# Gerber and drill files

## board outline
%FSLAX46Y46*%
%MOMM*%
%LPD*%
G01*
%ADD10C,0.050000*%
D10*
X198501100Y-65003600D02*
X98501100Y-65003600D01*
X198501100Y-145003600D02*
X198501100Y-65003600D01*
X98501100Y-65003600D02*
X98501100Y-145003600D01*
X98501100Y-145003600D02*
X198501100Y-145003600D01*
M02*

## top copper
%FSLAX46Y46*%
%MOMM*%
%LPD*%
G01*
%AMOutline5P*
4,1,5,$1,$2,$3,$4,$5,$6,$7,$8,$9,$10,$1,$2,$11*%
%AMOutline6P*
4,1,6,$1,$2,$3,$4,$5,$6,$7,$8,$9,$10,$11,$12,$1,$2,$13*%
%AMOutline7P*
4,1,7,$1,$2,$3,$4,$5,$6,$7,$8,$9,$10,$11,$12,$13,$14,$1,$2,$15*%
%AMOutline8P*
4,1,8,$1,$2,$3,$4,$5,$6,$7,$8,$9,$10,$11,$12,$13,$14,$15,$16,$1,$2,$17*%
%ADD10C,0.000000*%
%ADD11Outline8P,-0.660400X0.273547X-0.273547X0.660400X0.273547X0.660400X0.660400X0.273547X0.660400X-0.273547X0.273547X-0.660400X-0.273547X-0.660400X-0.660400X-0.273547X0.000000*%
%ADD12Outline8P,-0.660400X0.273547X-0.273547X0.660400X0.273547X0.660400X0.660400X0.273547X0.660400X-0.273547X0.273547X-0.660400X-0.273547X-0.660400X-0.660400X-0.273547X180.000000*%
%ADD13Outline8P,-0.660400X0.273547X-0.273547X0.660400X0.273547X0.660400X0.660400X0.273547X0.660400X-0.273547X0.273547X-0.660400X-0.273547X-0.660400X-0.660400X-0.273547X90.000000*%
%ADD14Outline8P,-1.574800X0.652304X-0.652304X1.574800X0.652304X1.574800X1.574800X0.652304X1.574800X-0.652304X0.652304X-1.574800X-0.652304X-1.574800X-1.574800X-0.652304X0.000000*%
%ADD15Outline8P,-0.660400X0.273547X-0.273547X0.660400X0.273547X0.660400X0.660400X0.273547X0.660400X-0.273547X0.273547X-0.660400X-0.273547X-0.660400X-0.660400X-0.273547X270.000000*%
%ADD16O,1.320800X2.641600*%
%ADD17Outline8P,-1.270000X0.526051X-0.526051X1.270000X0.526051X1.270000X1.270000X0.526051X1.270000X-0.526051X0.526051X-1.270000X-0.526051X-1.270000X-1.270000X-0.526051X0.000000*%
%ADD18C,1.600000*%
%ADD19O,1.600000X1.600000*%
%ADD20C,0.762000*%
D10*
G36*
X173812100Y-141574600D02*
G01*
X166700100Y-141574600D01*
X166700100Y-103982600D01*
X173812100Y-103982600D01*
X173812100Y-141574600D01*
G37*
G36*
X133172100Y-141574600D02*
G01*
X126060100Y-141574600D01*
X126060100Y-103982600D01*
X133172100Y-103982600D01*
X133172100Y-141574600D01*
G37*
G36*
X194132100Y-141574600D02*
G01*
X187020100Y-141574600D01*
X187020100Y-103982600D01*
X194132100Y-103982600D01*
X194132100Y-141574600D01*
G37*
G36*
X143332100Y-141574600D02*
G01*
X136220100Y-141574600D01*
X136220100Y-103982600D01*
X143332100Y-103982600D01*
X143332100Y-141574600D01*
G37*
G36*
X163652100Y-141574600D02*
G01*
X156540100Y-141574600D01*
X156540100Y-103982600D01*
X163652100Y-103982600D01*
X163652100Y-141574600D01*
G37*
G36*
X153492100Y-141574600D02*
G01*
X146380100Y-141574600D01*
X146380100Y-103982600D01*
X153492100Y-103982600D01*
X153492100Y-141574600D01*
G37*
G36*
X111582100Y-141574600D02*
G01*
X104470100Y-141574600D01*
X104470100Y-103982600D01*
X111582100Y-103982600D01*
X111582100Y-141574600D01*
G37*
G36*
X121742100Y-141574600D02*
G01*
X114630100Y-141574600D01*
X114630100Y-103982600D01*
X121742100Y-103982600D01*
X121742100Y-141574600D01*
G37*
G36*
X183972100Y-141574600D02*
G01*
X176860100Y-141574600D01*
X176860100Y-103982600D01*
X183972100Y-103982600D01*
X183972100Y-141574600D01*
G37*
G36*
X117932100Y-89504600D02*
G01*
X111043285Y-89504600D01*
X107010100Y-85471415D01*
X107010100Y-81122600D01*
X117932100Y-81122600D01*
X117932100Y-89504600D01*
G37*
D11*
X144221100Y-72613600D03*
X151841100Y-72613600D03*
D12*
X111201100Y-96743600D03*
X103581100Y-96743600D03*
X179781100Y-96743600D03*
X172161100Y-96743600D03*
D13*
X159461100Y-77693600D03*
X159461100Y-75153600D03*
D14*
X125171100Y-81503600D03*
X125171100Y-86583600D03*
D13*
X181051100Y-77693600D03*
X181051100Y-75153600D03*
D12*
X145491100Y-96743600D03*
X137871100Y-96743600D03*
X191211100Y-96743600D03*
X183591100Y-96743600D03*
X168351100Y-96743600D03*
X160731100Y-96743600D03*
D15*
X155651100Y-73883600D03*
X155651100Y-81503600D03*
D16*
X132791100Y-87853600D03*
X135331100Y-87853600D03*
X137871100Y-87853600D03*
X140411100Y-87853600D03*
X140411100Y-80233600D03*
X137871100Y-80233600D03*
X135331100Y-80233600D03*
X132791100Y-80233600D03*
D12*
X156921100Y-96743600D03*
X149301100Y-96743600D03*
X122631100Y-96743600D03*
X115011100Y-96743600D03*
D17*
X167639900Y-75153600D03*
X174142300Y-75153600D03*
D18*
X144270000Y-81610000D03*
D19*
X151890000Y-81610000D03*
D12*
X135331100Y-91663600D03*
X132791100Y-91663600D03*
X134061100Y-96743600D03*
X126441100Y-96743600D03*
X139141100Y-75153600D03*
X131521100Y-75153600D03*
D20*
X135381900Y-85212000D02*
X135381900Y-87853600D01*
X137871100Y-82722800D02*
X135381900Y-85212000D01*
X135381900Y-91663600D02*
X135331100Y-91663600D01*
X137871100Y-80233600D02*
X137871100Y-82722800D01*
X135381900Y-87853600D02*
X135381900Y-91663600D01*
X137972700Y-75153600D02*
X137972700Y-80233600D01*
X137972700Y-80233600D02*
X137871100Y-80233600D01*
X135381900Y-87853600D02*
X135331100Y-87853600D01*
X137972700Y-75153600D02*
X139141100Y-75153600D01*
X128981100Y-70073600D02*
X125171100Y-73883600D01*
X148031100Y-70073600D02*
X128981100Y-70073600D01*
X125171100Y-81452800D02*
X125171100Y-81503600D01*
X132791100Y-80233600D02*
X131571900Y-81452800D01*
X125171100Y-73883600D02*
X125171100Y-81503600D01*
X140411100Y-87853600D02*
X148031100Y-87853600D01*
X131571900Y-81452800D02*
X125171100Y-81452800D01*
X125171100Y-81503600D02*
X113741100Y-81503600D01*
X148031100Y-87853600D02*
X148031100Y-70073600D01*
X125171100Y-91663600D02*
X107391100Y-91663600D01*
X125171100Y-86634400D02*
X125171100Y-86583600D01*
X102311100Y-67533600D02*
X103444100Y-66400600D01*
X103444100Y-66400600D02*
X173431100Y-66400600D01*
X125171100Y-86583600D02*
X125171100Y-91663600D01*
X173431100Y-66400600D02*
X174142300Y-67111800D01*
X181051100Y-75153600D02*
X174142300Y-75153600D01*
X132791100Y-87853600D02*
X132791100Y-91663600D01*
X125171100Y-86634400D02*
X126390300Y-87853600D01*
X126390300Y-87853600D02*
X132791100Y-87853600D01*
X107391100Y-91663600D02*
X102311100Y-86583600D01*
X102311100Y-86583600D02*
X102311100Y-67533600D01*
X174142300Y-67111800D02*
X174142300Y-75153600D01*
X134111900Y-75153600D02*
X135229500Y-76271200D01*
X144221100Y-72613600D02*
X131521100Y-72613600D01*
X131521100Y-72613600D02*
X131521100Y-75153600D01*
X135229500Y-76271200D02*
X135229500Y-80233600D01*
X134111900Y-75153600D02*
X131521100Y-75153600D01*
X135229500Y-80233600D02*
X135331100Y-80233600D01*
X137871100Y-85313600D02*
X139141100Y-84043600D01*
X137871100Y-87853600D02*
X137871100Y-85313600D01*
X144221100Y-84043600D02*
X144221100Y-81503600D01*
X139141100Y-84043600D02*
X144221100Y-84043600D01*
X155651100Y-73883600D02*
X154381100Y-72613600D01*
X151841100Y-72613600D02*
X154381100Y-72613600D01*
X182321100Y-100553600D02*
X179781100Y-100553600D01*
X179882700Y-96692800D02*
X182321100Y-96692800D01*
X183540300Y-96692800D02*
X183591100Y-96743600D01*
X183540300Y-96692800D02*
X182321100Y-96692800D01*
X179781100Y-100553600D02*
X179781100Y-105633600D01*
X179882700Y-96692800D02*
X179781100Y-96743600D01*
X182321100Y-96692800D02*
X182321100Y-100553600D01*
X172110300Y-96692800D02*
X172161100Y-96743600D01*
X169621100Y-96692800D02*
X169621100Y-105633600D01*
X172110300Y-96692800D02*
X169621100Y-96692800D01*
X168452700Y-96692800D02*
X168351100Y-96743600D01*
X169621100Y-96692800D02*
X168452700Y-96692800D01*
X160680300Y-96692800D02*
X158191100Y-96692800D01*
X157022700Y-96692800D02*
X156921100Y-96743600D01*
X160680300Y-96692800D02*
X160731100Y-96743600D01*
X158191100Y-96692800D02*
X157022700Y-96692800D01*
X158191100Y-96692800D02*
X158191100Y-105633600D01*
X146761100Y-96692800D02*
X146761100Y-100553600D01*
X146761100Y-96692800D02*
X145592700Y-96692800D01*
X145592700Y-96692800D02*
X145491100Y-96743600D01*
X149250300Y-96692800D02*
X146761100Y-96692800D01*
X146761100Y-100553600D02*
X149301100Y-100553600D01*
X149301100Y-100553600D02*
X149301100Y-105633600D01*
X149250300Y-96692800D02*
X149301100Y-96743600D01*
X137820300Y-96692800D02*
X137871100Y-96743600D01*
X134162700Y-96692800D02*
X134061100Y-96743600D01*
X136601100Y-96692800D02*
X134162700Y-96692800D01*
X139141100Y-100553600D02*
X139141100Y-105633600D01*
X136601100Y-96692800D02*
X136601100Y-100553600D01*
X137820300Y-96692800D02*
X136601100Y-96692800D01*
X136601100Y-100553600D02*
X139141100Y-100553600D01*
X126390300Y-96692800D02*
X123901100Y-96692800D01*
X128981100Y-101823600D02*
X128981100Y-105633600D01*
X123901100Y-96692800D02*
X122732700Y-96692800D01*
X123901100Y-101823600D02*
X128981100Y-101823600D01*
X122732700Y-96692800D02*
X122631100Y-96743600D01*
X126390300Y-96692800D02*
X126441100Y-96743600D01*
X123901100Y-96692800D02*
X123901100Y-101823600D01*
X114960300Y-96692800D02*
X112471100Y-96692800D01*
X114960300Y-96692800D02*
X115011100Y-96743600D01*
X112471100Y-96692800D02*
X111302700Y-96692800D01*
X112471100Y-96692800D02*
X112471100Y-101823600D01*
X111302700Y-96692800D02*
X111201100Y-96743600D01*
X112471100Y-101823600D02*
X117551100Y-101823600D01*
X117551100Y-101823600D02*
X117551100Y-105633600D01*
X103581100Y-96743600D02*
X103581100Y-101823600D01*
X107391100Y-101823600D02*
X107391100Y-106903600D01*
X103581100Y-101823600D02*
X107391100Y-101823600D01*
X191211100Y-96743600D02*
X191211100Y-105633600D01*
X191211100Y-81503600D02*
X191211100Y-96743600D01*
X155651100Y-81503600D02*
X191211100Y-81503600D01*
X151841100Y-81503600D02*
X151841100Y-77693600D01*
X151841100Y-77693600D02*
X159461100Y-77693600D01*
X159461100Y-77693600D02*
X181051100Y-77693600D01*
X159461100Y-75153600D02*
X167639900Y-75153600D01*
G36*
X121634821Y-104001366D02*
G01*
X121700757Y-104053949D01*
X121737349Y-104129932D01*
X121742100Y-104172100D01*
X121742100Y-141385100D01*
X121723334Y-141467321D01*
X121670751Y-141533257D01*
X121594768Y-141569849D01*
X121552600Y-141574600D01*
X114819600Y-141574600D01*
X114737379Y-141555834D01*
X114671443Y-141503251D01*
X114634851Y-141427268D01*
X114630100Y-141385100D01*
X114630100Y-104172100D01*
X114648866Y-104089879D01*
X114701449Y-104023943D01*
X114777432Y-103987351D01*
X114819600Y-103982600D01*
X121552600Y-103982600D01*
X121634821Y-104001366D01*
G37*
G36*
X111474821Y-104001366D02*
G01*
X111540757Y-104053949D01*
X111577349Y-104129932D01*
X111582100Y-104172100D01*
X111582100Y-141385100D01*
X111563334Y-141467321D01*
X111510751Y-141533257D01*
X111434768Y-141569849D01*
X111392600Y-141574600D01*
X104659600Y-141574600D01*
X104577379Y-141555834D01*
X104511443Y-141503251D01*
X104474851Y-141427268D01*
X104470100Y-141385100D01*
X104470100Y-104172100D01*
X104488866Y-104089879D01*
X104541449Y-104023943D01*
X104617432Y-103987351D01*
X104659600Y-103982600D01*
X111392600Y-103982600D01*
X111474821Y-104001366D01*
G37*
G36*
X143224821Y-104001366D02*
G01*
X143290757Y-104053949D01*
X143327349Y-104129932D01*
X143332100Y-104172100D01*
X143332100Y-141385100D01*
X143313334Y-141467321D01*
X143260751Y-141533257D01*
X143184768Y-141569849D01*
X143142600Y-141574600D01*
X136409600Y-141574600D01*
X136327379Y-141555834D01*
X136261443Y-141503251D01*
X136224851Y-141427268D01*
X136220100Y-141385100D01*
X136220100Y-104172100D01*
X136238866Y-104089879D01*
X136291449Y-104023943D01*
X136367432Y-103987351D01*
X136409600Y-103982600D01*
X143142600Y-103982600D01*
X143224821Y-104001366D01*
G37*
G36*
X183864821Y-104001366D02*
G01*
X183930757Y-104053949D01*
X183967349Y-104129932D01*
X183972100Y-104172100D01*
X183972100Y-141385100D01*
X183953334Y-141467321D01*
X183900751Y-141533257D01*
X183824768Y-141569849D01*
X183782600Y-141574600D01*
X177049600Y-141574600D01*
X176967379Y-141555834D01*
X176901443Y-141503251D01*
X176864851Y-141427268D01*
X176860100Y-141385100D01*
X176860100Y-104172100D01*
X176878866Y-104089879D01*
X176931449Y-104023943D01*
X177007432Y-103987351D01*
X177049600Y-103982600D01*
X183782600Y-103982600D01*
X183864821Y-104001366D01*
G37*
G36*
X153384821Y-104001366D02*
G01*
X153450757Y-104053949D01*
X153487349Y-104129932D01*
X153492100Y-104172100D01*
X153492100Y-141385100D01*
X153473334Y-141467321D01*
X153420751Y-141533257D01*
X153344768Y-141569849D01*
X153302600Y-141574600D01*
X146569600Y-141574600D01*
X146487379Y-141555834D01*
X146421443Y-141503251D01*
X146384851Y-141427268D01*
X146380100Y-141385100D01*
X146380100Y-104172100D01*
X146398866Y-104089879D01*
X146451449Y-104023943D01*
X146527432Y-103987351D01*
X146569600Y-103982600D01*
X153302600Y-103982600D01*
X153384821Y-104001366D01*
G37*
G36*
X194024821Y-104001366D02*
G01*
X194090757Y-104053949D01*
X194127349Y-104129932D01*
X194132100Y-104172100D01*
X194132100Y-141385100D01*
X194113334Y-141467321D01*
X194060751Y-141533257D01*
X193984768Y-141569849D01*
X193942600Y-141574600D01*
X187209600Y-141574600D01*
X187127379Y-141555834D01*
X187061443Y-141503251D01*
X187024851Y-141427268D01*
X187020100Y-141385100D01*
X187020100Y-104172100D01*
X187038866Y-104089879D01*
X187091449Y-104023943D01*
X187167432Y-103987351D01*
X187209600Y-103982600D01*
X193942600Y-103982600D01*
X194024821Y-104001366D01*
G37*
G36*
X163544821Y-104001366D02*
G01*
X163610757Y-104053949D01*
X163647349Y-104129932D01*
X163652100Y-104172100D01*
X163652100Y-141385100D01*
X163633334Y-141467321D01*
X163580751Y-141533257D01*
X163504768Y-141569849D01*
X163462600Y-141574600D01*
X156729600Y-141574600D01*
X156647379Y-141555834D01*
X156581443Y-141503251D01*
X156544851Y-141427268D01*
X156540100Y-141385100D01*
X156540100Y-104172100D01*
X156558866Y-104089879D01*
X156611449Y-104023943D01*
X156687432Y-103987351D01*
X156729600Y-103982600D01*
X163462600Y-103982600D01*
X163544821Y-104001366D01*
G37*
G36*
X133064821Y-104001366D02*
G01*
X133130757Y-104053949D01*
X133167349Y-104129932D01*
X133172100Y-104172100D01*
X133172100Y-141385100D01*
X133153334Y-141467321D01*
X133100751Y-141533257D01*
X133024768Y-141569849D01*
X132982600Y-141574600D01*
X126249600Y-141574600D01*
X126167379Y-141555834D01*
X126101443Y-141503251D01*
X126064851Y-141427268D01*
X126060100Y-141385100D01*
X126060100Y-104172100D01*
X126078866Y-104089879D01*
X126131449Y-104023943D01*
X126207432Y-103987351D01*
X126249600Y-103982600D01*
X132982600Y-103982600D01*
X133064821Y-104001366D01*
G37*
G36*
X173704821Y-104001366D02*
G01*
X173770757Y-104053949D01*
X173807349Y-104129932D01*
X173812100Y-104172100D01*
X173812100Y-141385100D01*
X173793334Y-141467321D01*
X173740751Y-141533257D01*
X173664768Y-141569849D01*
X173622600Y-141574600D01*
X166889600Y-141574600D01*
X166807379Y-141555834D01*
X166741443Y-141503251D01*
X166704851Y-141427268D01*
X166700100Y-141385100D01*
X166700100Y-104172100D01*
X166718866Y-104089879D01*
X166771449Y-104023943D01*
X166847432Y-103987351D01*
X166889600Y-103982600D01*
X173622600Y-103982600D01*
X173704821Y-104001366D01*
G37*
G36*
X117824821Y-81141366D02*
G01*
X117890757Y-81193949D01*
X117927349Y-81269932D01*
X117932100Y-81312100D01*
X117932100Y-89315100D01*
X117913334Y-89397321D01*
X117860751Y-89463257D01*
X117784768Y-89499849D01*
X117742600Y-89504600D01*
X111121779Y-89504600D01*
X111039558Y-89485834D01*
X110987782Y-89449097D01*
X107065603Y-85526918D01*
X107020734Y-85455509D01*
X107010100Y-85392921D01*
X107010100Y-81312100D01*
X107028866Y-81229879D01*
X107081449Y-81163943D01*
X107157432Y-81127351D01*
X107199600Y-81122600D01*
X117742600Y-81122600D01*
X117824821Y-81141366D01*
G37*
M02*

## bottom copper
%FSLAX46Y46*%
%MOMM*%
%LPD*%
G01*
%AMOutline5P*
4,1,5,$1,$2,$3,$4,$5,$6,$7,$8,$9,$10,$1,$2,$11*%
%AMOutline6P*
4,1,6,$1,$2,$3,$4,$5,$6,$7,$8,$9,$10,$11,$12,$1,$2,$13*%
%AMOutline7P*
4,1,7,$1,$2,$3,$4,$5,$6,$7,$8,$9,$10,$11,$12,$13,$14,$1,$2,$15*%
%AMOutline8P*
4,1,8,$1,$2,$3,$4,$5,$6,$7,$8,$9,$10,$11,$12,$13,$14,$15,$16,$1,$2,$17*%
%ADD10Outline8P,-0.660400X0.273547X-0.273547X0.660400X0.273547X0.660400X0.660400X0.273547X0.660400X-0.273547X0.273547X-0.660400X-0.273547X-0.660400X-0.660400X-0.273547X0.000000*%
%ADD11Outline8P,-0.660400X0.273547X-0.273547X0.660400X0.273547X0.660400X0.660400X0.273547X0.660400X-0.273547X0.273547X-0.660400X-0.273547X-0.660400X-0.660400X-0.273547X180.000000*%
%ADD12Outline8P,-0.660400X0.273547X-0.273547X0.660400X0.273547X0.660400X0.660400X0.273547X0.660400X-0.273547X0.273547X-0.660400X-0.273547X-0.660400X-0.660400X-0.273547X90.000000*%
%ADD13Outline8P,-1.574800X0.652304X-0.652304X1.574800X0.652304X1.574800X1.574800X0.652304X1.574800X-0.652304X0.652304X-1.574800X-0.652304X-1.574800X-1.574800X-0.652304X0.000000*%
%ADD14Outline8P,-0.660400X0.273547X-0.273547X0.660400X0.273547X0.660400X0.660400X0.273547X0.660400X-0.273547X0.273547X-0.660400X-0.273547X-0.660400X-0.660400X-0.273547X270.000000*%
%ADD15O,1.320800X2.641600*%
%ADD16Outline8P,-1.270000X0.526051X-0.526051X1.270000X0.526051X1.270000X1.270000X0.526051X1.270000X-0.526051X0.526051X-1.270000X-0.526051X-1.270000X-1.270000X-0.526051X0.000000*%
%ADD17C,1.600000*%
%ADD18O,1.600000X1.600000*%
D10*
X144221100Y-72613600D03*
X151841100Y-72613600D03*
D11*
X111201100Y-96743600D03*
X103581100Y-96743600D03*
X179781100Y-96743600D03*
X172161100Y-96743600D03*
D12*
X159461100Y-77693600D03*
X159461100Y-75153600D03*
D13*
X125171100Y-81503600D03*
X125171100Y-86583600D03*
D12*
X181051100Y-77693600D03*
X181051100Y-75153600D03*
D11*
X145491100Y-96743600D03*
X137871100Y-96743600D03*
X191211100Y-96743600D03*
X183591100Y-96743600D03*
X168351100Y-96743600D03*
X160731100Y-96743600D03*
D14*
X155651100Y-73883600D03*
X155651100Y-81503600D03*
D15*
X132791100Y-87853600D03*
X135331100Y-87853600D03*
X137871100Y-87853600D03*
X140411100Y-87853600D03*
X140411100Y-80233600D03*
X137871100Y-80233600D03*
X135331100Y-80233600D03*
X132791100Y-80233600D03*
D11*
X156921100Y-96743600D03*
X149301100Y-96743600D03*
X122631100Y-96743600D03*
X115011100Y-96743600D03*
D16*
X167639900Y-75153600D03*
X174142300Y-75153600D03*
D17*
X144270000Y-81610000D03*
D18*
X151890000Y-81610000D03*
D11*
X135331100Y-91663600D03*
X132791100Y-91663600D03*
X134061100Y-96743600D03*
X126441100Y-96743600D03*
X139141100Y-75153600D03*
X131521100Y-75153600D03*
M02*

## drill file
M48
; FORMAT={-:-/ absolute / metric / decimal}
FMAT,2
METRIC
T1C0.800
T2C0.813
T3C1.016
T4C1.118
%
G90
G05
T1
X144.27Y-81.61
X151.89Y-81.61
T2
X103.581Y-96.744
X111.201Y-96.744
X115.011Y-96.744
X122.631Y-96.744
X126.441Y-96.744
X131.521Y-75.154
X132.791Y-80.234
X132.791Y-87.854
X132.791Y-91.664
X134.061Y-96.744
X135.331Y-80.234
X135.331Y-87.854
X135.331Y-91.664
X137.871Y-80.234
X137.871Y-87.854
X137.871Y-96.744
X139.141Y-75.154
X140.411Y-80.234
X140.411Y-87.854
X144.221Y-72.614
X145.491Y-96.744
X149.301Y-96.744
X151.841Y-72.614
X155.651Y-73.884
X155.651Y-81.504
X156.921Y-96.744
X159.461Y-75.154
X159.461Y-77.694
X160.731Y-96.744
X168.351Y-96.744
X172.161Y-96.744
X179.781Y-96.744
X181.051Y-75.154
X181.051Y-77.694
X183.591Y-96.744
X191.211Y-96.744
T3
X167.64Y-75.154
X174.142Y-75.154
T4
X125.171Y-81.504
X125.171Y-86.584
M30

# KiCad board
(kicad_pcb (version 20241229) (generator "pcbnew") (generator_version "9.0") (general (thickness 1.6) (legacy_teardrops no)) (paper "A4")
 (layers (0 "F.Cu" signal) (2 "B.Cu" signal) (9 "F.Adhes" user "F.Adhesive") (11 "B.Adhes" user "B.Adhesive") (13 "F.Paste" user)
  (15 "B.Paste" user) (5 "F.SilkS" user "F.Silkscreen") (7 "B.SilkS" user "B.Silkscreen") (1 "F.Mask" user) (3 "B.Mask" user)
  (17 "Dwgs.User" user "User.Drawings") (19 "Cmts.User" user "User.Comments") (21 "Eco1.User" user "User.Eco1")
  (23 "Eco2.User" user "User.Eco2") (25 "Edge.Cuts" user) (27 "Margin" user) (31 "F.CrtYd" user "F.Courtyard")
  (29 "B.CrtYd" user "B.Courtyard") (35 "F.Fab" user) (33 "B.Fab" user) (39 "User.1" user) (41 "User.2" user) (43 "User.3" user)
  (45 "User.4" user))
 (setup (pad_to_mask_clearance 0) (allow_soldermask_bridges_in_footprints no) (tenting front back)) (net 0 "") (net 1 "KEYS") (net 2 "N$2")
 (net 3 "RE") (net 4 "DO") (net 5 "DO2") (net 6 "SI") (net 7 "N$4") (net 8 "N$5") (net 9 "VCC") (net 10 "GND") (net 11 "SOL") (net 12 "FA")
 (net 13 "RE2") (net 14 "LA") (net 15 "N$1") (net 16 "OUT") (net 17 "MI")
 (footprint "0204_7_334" (layer "F.Cu") (at 148.0311 72.6136)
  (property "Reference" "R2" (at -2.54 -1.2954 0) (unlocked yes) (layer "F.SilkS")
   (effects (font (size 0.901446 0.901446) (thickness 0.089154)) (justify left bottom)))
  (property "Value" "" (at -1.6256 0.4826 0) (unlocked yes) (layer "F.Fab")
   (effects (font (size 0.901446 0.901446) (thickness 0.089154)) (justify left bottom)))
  (pad "1" thru_hole roundrect (at -3.81 0) (size 1.3208 1.3208) (drill 0.8128) (layers "*.Cu" "*.Mask") (remove_unused_layers no)
   (roundrect_rratio 0.25) (chamfer_ratio 0.2928932188) (chamfer top_left top_right bottom_left bottom_right) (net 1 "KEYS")
   (solder_mask_margin 0.1016) (thermal_bridge_angle 0))
  (pad "2" thru_hole roundrect (at 3.81 0) (size 1.3208 1.3208) (drill 0.8128) (layers "*.Cu" "*.Mask") (remove_unused_layers no)
   (roundrect_rratio 0.25) (chamfer_ratio 0.2928932188) (chamfer top_left top_right bottom_left bottom_right) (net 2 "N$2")
   (solder_mask_margin 0.1016) (thermal_bridge_angle 0)))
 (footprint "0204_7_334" (layer "F.Cu") (at 107.3911 96.7436 180)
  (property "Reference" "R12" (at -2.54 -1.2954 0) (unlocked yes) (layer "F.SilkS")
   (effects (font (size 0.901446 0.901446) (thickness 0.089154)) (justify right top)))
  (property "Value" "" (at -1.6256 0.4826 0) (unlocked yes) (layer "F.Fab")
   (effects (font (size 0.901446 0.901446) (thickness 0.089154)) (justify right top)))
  (pad "1" thru_hole roundrect (at -3.81 0 180) (size 1.3208 1.3208) (drill 0.8128) (layers "*.Cu" "*.Mask") (remove_unused_layers no)
   (roundrect_rratio 0.25) (chamfer_ratio 0.2928932188) (chamfer top_left top_right bottom_left bottom_right) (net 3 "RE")
   (solder_mask_margin 0.1016) (thermal_bridge_angle 0))
  (pad "2" thru_hole roundrect (at 3.81 0 180) (size 1.3208 1.3208) (drill 0.8128) (layers "*.Cu" "*.Mask") (remove_unused_layers no)
   (roundrect_rratio 0.25) (chamfer_ratio 0.2928932188) (chamfer top_left top_right bottom_left bottom_right) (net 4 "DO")
   (solder_mask_margin 0.1016) (thermal_bridge_angle 0)))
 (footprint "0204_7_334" (layer "F.Cu") (at 175.9711 96.7436 180)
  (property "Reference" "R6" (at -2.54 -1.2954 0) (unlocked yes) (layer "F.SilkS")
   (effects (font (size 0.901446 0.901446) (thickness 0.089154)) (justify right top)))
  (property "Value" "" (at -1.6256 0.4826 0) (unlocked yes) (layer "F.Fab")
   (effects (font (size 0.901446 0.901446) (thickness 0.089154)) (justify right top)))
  (pad "1" thru_hole roundrect (at -3.81 0 180) (size 1.3208 1.3208) (drill 0.8128) (layers "*.Cu" "*.Mask") (remove_unused_layers no)
   (roundrect_rratio 0.25) (chamfer_ratio 0.2928932188) (chamfer top_left top_right bottom_left bottom_right) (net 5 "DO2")
   (solder_mask_margin 0.1016) (thermal_bridge_angle 0))
  (pad "2" thru_hole roundrect (at 3.81 0 180) (size 1.3208 1.3208) (drill 0.8128) (layers "*.Cu" "*.Mask") (remove_unused_layers no)
   (roundrect_rratio 0.25) (chamfer_ratio 0.2928932188) (chamfer top_left top_right bottom_left bottom_right) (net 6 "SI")
   (solder_mask_margin 0.1016) (thermal_bridge_angle 0)))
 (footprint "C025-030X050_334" (layer "F.Cu") (at 159.4611 76.4236 90)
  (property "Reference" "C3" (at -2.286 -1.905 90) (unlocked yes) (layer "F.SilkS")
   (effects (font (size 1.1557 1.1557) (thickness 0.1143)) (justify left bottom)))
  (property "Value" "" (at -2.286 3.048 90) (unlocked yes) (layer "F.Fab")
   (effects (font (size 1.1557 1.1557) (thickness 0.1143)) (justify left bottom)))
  (pad "1" thru_hole roundrect (at -1.27 0 90) (size 1.3208 1.3208) (drill 0.8128) (layers "*.Cu" "*.Mask") (remove_unused_layers no)
   (roundrect_rratio 0.25) (chamfer_ratio 0.2928932188) (chamfer top_left top_right bottom_left bottom_right) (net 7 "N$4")
   (solder_mask_margin 0.1016) (thermal_bridge_angle 0))
  (pad "2" thru_hole roundrect (at 1.27 0 90) (size 1.3208 1.3208) (drill 0.8128) (layers "*.Cu" "*.Mask") (remove_unused_layers no)
   (roundrect_rratio 0.25) (chamfer_ratio 0.2928932188) (chamfer top_left top_right bottom_left bottom_right) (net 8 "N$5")
   (solder_mask_margin 0.1016) (thermal_bridge_angle 0)))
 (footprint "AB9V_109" (layer "F.Cu") (at 125.1711 84.0436)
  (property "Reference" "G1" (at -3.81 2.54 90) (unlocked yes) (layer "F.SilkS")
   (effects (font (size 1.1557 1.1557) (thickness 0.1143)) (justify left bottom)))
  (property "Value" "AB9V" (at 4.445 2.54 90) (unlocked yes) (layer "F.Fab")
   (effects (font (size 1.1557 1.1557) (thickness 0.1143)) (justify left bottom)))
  (pad "+" thru_hole roundrect (at 0 -2.54) (size 3.1496 3.1496) (drill 1.1176) (layers "*.Cu" "*.Mask") (remove_unused_layers no)
   (roundrect_rratio 0.25) (chamfer_ratio 0.2928932188) (chamfer top_left top_right bottom_left bottom_right) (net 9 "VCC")
   (solder_mask_margin 0.1016) (thermal_bridge_angle 0))
  (pad "-" thru_hole roundrect (at 0 2.54) (size 3.1496 3.1496) (drill 1.1176) (layers "*.Cu" "*.Mask") (remove_unused_layers no)
   (roundrect_rratio 0.25) (chamfer_ratio 0.2928932188) (chamfer top_left top_right bottom_left bottom_right) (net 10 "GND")
   (solder_mask_margin 0.1016) (thermal_bridge_angle 0)))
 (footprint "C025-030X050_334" (layer "F.Cu") (at 181.0511 76.4236 90)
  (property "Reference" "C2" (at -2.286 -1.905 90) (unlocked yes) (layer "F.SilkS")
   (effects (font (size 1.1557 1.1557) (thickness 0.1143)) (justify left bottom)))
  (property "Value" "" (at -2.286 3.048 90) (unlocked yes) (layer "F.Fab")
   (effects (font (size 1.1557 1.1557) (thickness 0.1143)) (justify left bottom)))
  (pad "1" thru_hole roundrect (at -1.27 0 90) (size 1.3208 1.3208) (drill 0.8128) (layers "*.Cu" "*.Mask") (remove_unused_layers no)
   (roundrect_rratio 0.25) (chamfer_ratio 0.2928932188) (chamfer top_left top_right bottom_left bottom_right) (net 7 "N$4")
   (solder_mask_margin 0.1016) (thermal_bridge_angle 0))
  (pad "2" thru_hole roundrect (at 1.27 0 90) (size 1.3208 1.3208) (drill 0.8128) (layers "*.Cu" "*.Mask") (remove_unused_layers no)
   (roundrect_rratio 0.25) (chamfer_ratio 0.2928932188) (chamfer top_left top_right bottom_left bottom_right) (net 10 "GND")
   (solder_mask_margin 0.1016) (thermal_bridge_angle 0)))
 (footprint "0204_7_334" (layer "F.Cu") (at 141.6811 96.7436 180)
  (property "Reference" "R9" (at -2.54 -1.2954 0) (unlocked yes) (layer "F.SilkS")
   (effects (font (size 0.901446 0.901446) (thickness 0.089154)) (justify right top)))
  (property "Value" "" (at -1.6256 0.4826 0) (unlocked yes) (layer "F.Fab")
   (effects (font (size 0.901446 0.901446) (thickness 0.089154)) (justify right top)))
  (pad "1" thru_hole roundrect (at -3.81 0 180) (size 1.3208 1.3208) (drill 0.8128) (layers "*.Cu" "*.Mask") (remove_unused_layers no)
   (roundrect_rratio 0.25) (chamfer_ratio 0.2928932188) (chamfer top_left top_right bottom_left bottom_right) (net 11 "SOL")
   (solder_mask_margin 0.1016) (thermal_bridge_angle 0))
  (pad "2" thru_hole roundrect (at 3.81 0 180) (size 1.3208 1.3208) (drill 0.8128) (layers "*.Cu" "*.Mask") (remove_unused_layers no)
   (roundrect_rratio 0.25) (chamfer_ratio 0.2928932188) (chamfer top_left top_right bottom_left bottom_right) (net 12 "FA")
   (solder_mask_margin 0.1016) (thermal_bridge_angle 0)))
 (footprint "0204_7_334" (layer "F.Cu") (at 187.4011 96.7436 180)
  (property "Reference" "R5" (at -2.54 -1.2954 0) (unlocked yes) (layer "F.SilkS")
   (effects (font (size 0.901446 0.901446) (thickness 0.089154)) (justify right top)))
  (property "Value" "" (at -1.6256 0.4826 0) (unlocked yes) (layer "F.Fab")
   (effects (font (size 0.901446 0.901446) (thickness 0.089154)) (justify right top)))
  (pad "1" thru_hole roundrect (at -3.81 0 180) (size 1.3208 1.3208) (drill 0.8128) (layers "*.Cu" "*.Mask") (remove_unused_layers no)
   (roundrect_rratio 0.25) (chamfer_ratio 0.2928932188) (chamfer top_left top_right bottom_left bottom_right) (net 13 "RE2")
   (solder_mask_margin 0.1016) (thermal_bridge_angle 0))
  (pad "2" thru_hole roundrect (at 3.81 0 180) (size 1.3208 1.3208) (drill 0.8128) (layers "*.Cu" "*.Mask") (remove_unused_layers no)
   (roundrect_rratio 0.25) (chamfer_ratio 0.2928932188) (chamfer top_left top_right bottom_left bottom_right) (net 5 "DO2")
   (solder_mask_margin 0.1016) (thermal_bridge_angle 0)))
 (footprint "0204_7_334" (layer "F.Cu") (at 164.5411 96.7436 180)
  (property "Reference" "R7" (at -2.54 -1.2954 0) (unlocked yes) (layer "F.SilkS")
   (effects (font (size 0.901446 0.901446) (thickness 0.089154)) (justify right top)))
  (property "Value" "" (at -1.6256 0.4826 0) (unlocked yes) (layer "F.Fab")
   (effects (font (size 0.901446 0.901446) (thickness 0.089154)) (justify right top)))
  (pad "1" thru_hole roundrect (at -3.81 0 180) (size 1.3208 1.3208) (drill 0.8128) (layers "*.Cu" "*.Mask") (remove_unused_layers no)
   (roundrect_rratio 0.25) (chamfer_ratio 0.2928932188) (chamfer top_left top_right bottom_left bottom_right) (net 6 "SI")
   (solder_mask_margin 0.1016) (thermal_bridge_angle 0))
  (pad "2" thru_hole roundrect (at 3.81 0 180) (size 1.3208 1.3208) (drill 0.8128) (layers "*.Cu" "*.Mask") (remove_unused_layers no)
   (roundrect_rratio 0.25) (chamfer_ratio 0.2928932188) (chamfer top_left top_right bottom_left bottom_right) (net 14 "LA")
   (solder_mask_margin 0.1016) (thermal_bridge_angle 0)))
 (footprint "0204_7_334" (layer "F.Cu") (at 155.6511 77.6936 -90)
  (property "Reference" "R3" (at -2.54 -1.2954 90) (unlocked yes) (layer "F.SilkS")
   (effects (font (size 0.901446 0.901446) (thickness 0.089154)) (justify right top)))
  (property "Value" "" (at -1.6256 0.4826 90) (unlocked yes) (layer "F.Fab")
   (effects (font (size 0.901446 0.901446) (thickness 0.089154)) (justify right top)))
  (pad "1" thru_hole roundrect (at -3.81 0 270) (size 1.3208 1.3208) (drill 0.8128) (layers "*.Cu" "*.Mask") (remove_unused_layers no)
   (roundrect_rratio 0.25) (chamfer_ratio 0.2928932188) (chamfer top_left top_right bottom_left bottom_right) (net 2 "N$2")
   (solder_mask_margin 0.1016) (thermal_bridge_angle 0))
  (pad "2" thru_hole roundrect (at 3.81 0 270) (size 1.3208 1.3208) (drill 0.8128) (layers "*.Cu" "*.Mask") (remove_unused_layers no)
   (roundrect_rratio 0.25) (chamfer_ratio 0.2928932188) (chamfer top_left top_right bottom_left bottom_right) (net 13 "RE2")
   (solder_mask_margin 0.1016) (thermal_bridge_angle 0)))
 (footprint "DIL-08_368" (layer "F.Cu") (at 136.6011 84.0436)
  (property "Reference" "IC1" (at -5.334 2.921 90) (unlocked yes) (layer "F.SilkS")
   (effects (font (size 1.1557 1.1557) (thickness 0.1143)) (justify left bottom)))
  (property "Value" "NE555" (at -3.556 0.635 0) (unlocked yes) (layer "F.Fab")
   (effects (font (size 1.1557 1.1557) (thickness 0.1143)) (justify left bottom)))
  (pad "1" thru_hole oval (at -3.81 3.81 90) (size 2.6416 1.3208) (drill 0.8128) (layers "*.Cu" "*.Mask") (remove_unused_layers no)
   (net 10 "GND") (solder_mask_margin 0.1016) (thermal_bridge_angle 0))
  (pad "2" thru_hole oval (at -1.27 3.81 90) (size 2.6416 1.3208) (drill 0.8128) (layers "*.Cu" "*.Mask") (remove_unused_layers no)
   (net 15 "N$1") (solder_mask_margin 0.1016) (thermal_bridge_angle 0))
  (pad "3" thru_hole oval (at 1.27 3.81 90) (size 2.6416 1.3208) (drill 0.8128) (layers "*.Cu" "*.Mask") (remove_unused_layers no)
   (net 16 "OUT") (solder_mask_margin 0.1016) (thermal_bridge_angle 0))
  (pad "4" thru_hole oval (at 3.81 3.81 90) (size 2.6416 1.3208) (drill 0.8128) (layers "*.Cu" "*.Mask") (remove_unused_layers no)
   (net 9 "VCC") (solder_mask_margin 0.1016) (thermal_bridge_angle 0))
  (pad "5" thru_hole oval (at 3.81 -3.81 90) (size 2.6416 1.3208) (drill 0.8128) (layers "*.Cu" "*.Mask") (remove_unused_layers no)
   (solder_mask_margin 0.1016) (thermal_bridge_angle 0))
  (pad "6" thru_hole oval (at 1.27 -3.81 90) (size 2.6416 1.3208) (drill 0.8128) (layers "*.Cu" "*.Mask") (remove_unused_layers no)
   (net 15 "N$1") (solder_mask_margin 0.1016) (thermal_bridge_angle 0))
  (pad "7" thru_hole oval (at -1.27 -3.81 90) (size 2.6416 1.3208) (drill 0.8128) (layers "*.Cu" "*.Mask") (remove_unused_layers no)
   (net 1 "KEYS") (solder_mask_margin 0.1016) (thermal_bridge_angle 0))
  (pad "8" thru_hole oval (at -3.81 -3.81 90) (size 2.6416 1.3208) (drill 0.8128) (layers "*.Cu" "*.Mask") (remove_unused_layers no)
   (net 9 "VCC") (solder_mask_margin 0.1016) (thermal_bridge_angle 0)))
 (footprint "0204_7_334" (layer "F.Cu") (at 153.1111 96.7436 180)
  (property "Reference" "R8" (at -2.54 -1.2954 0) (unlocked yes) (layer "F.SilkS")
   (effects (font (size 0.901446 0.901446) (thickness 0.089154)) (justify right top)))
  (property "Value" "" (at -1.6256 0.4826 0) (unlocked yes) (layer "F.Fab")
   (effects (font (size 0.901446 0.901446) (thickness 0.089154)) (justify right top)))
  (pad "1" thru_hole roundrect (at -3.81 0 180) (size 1.3208 1.3208) (drill 0.8128) (layers "*.Cu" "*.Mask") (remove_unused_layers no)
   (roundrect_rratio 0.25) (chamfer_ratio 0.2928932188) (chamfer top_left top_right bottom_left bottom_right) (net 14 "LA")
   (solder_mask_margin 0.1016) (thermal_bridge_angle 0))
  (pad "2" thru_hole roundrect (at 3.81 0 180) (size 1.3208 1.3208) (drill 0.8128) (layers "*.Cu" "*.Mask") (remove_unused_layers no)
   (roundrect_rratio 0.25) (chamfer_ratio 0.2928932188) (chamfer top_left top_right bottom_left bottom_right) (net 11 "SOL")
   (solder_mask_margin 0.1016) (thermal_bridge_angle 0)))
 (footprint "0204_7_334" (layer "F.Cu") (at 118.8211 96.7436 180)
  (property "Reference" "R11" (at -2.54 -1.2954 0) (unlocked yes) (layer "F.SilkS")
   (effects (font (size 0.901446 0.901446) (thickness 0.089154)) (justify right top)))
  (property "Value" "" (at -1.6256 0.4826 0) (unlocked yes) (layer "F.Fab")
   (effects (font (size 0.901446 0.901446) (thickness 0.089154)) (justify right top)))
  (pad "1" thru_hole roundrect (at -3.81 0 180) (size 1.3208 1.3208) (drill 0.8128) (layers "*.Cu" "*.Mask") (remove_unused_layers no)
   (roundrect_rratio 0.25) (chamfer_ratio 0.2928932188) (chamfer top_left top_right bottom_left bottom_right) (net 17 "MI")
   (solder_mask_margin 0.1016) (thermal_bridge_angle 0))
  (pad "2" thru_hole roundrect (at 3.81 0 180) (size 1.3208 1.3208) (drill 0.8128) (layers "*.Cu" "*.Mask") (remove_unused_layers no)
   (roundrect_rratio 0.25) (chamfer_ratio 0.2928932188) (chamfer top_left top_right bottom_left bottom_right) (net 3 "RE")
   (solder_mask_margin 0.1016) (thermal_bridge_angle 0)))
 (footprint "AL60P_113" (layer "F.Cu") (at 170.8911 75.1536)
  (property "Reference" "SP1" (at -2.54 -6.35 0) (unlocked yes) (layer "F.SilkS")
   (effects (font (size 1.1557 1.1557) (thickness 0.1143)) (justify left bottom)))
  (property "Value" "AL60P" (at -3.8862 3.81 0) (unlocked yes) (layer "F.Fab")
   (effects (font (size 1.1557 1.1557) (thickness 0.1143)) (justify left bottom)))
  (pad "1" thru_hole roundrect (at -3.2512 0) (size 2.54 2.54) (drill 1.016) (layers "*.Cu" "*.Mask") (remove_unused_layers no)
   (roundrect_rratio 0.25) (chamfer_ratio 0.2928932188) (chamfer top_left top_right bottom_left bottom_right) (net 8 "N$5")
   (solder_mask_margin 0.1016) (thermal_bridge_angle 0))
  (pad "2" thru_hole roundrect (at 3.2512 0) (size 2.54 2.54) (drill 1.016) (layers "*.Cu" "*.Mask") (remove_unused_layers no)
   (roundrect_rratio 0.25) (chamfer_ratio 0.2928932188) (chamfer top_left top_right bottom_left bottom_right) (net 10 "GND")
   (solder_mask_margin 0.1016) (thermal_bridge_angle 0)))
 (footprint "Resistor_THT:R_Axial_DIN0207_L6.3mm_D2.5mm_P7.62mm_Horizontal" (layer "F.Cu") (at 144.27 81.61)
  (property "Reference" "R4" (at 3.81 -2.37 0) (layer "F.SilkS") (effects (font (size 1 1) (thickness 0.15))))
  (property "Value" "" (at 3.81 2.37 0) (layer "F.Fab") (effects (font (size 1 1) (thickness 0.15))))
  (pad "1" thru_hole circle (at 0 0) (size 1.6 1.6) (drill 0.8) (layers "*.Cu" "*.Mask") (remove_unused_layers no) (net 16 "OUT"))
  (pad "2" thru_hole oval (at 7.62 0) (size 1.6 1.6) (drill 0.8) (layers "*.Cu" "*.Mask") (remove_unused_layers no) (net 7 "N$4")))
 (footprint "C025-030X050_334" (layer "F.Cu") (at 134.0611 91.6636 180)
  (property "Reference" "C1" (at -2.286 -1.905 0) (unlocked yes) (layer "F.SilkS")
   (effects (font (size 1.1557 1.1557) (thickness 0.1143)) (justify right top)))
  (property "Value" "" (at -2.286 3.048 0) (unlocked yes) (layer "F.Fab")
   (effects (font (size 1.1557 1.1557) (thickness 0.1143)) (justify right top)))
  (pad "1" thru_hole roundrect (at -1.27 0 180) (size 1.3208 1.3208) (drill 0.8128) (layers "*.Cu" "*.Mask") (remove_unused_layers no)
   (roundrect_rratio 0.25) (chamfer_ratio 0.2928932188) (chamfer top_left top_right bottom_left bottom_right) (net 15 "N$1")
   (solder_mask_margin 0.1016) (thermal_bridge_angle 0))
  (pad "2" thru_hole roundrect (at 1.27 0 180) (size 1.3208 1.3208) (drill 0.8128) (layers "*.Cu" "*.Mask") (remove_unused_layers no)
   (roundrect_rratio 0.25) (chamfer_ratio 0.2928932188) (chamfer top_left top_right bottom_left bottom_right) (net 10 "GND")
   (solder_mask_margin 0.1016) (thermal_bridge_angle 0)))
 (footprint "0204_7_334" (layer "F.Cu") (at 130.2511 96.7436 180)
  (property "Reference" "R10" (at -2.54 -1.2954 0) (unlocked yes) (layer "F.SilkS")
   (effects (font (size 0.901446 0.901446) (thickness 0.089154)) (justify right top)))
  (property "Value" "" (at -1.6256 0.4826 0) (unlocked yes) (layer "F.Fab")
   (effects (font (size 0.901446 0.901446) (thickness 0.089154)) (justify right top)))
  (pad "1" thru_hole roundrect (at -3.81 0 180) (size 1.3208 1.3208) (drill 0.8128) (layers "*.Cu" "*.Mask") (remove_unused_layers no)
   (roundrect_rratio 0.25) (chamfer_ratio 0.2928932188) (chamfer top_left top_right bottom_left bottom_right) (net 12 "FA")
   (solder_mask_margin 0.1016) (thermal_bridge_angle 0))
  (pad "2" thru_hole roundrect (at 3.81 0 180) (size 1.3208 1.3208) (drill 0.8128) (layers "*.Cu" "*.Mask") (remove_unused_layers no)
   (roundrect_rratio 0.25) (chamfer_ratio 0.2928932188) (chamfer top_left top_right bottom_left bottom_right) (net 17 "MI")
   (solder_mask_margin 0.1016) (thermal_bridge_angle 0)))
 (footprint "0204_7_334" (layer "F.Cu") (at 135.3311 75.1536 180)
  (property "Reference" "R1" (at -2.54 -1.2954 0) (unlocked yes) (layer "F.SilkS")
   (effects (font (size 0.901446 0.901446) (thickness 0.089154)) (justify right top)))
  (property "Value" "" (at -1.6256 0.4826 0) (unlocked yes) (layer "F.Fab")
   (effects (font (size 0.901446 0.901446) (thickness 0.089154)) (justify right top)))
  (pad "1" thru_hole roundrect (at -3.81 0 180) (size 1.3208 1.3208) (drill 0.8128) (layers "*.Cu" "*.Mask") (remove_unused_layers no)
   (roundrect_rratio 0.25) (chamfer_ratio 0.2928932188) (chamfer top_left top_right bottom_left bottom_right) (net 15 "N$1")
   (solder_mask_margin 0.1016) (thermal_bridge_angle 0))
  (pad "2" thru_hole roundrect (at 3.81 0 180) (size 1.3208 1.3208) (drill 0.8128) (layers "*.Cu" "*.Mask") (remove_unused_layers no)
   (roundrect_rratio 0.25) (chamfer_ratio 0.2928932188) (chamfer top_left top_right bottom_left bottom_right) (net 1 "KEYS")
   (solder_mask_margin 0.1016) (thermal_bridge_angle 0)))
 (gr_poly
  (pts (xy 173.8121 141.5746) (xy 166.7001 141.5746) (xy 166.7001 103.9826) (xy 173.8121 103.9826)) (stroke (width 0) (type solid))
  (fill yes) (layers "F.Cu" "F.Mask") (net 6))
 (gr_poly
  (pts (xy 133.1721 141.5746) (xy 126.0601 141.5746) (xy 126.0601 103.9826) (xy 133.1721 103.9826)) (stroke (width 0) (type solid))
  (fill yes) (layers "F.Cu" "F.Mask") (net 17))
 (gr_poly
  (pts (xy 194.1321 141.5746) (xy 187.0201 141.5746) (xy 187.0201 103.9826) (xy 194.1321 103.9826)) (stroke (width 0) (type solid))
  (fill yes) (layers "F.Cu" "F.Mask") (net 13))
 (gr_poly
  (pts (xy 143.3321 141.5746) (xy 136.2201 141.5746) (xy 136.2201 103.9826) (xy 143.3321 103.9826)) (stroke (width 0) (type solid))
  (fill yes) (layers "F.Cu" "F.Mask") (net 12))
 (gr_poly
  (pts (xy 163.6521 141.5746) (xy 156.5401 141.5746) (xy 156.5401 103.9826) (xy 163.6521 103.9826)) (stroke (width 0) (type solid))
  (fill yes) (layers "F.Cu" "F.Mask") (net 14))
 (gr_poly
  (pts (xy 153.4921 141.5746) (xy 146.3801 141.5746) (xy 146.3801 103.9826) (xy 153.4921 103.9826)) (stroke (width 0) (type solid))
  (fill yes) (layers "F.Cu" "F.Mask") (net 11))
 (gr_poly
  (pts (xy 111.5821 141.5746) (xy 104.4701 141.5746) (xy 104.4701 103.9826) (xy 111.5821 103.9826)) (stroke (width 0) (type solid))
  (fill yes) (layers "F.Cu" "F.Mask") (net 4))
 (gr_poly
  (pts (xy 121.7421 141.5746) (xy 114.6301 141.5746) (xy 114.6301 103.9826) (xy 121.7421 103.9826)) (stroke (width 0) (type solid))
  (fill yes) (layers "F.Cu" "F.Mask") (net 3))
 (gr_poly
  (pts (xy 183.9721 141.5746) (xy 176.8601 141.5746) (xy 176.8601 103.9826) (xy 183.9721 103.9826)) (stroke (width 0) (type solid))
  (fill yes) (layers "F.Cu" "F.Mask") (net 5))
 (gr_poly
  (pts (xy 117.9321 89.5046) (xy 111.043285 89.5046) (xy 107.0101 85.471415) (xy 107.0101 81.1226) (xy 117.9321 81.1226))
  (stroke (width 0) (type solid)) (fill yes) (layers "F.Cu" "F.Mask") (net 9))
 (gr_line (start 198.5011 65.0036) (end 98.5011 65.0036) (stroke (width 0.05) (type solid)) (layer "Edge.Cuts"))
 (gr_line (start 198.5011 145.0036) (end 198.5011 65.0036) (stroke (width 0.05) (type solid)) (layer "Edge.Cuts"))
 (gr_line (start 98.5011 65.0036) (end 98.5011 145.0036) (stroke (width 0.05) (type solid)) (layer "Edge.Cuts"))
 (gr_line (start 98.5011 145.0036) (end 198.5011 145.0036) (stroke (width 0.05) (type solid)) (layer "Edge.Cuts"))
 (segment (start 135.3819 85.212) (end 135.3819 87.8536) (width 0.762) (layer "F.Cu") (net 15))
 (segment (start 137.8711 82.7228) (end 135.3819 85.212) (width 0.762) (layer "F.Cu") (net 15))
 (segment (start 135.3819 91.6636) (end 135.3311 91.6636) (width 0.762) (layer "F.Cu") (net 15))
 (segment (start 137.8711 80.2336) (end 137.8711 82.7228) (width 0.762) (layer "F.Cu") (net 15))
 (segment (start 135.3819 87.8536) (end 135.3819 91.6636) (width 0.762) (layer "F.Cu") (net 15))
 (segment (start 137.9727 75.1536) (end 137.9727 80.2336) (width 0.762) (layer "F.Cu") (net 15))
 (segment (start 137.9727 80.2336) (end 137.8711 80.2336) (width 0.762) (layer "F.Cu") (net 15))
 (segment (start 135.3819 87.8536) (end 135.3311 87.8536) (width 0.762) (layer "F.Cu") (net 15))
 (segment (start 137.9727 75.1536) (end 139.1411 75.1536) (width 0.762) (layer "F.Cu") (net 15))
 (segment (start 128.9811 70.0736) (end 125.1711 73.8836) (width 0.762) (layer "F.Cu") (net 9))
 (segment (start 148.0311 70.0736) (end 128.9811 70.0736) (width 0.762) (layer "F.Cu") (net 9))
 (segment (start 125.1711 81.4528) (end 125.1711 81.5036) (width 0.762) (layer "F.Cu") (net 9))
 (segment (start 132.7911 80.2336) (end 131.5719 81.4528) (width 0.762) (layer "F.Cu") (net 9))
 (segment (start 125.1711 73.8836) (end 125.1711 81.5036) (width 0.762) (layer "F.Cu") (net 9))
 (segment (start 140.4111 87.8536) (end 148.0311 87.8536) (width 0.762) (layer "F.Cu") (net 9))
 (segment (start 131.5719 81.4528) (end 125.1711 81.4528) (width 0.762) (layer "F.Cu") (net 9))
 (segment (start 125.1711 81.5036) (end 113.7411 81.5036) (width 0.762) (layer "F.Cu") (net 9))
 (segment (start 148.0311 87.8536) (end 148.0311 70.0736) (width 0.762) (layer "F.Cu") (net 9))
 (segment (start 125.1711 91.6636) (end 107.3911 91.6636) (width 0.762) (layer "F.Cu") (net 10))
 (segment (start 125.1711 86.6344) (end 125.1711 86.5836) (width 0.762) (layer "F.Cu") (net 10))
 (segment (start 102.3111 67.5336) (end 103.4441 66.4006) (width 0.762) (layer "F.Cu") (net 10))
 (segment (start 103.4441 66.4006) (end 173.4311 66.4006) (width 0.762) (layer "F.Cu") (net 10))
 (segment (start 125.1711 86.5836) (end 125.1711 91.6636) (width 0.762) (layer "F.Cu") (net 10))
 (segment (start 173.4311 66.4006) (end 174.1423 67.1118) (width 0.762) (layer "F.Cu") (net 10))
 (segment (start 181.0511 75.1536) (end 174.1423 75.1536) (width 0.762) (layer "F.Cu") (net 10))
 (segment (start 132.7911 87.8536) (end 132.7911 91.6636) (width 0.762) (layer "F.Cu") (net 10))
 (segment (start 125.1711 86.6344) (end 126.3903 87.8536) (width 0.762) (layer "F.Cu") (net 10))
 (segment (start 126.3903 87.8536) (end 132.7911 87.8536) (width 0.762) (layer "F.Cu") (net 10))
 (segment (start 107.3911 91.6636) (end 102.3111 86.5836) (width 0.762) (layer "F.Cu") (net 10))
 (segment (start 102.3111 86.5836) (end 102.3111 67.5336) (width 0.762) (layer "F.Cu") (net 10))
 (segment (start 174.1423 67.1118) (end 174.1423 75.1536) (width 0.762) (layer "F.Cu") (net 10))
 (segment (start 134.1119 75.1536) (end 135.2295 76.2712) (width 0.762) (layer "F.Cu") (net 1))
 (segment (start 144.2211 72.6136) (end 131.5211 72.6136) (width 0.762) (layer "F.Cu") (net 1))
 (segment (start 131.5211 72.6136) (end 131.5211 75.1536) (width 0.762) (layer "F.Cu") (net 1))
 (segment (start 135.2295 76.2712) (end 135.2295 80.2336) (width 0.762) (layer "F.Cu") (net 1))
 (segment (start 134.1119 75.1536) (end 131.5211 75.1536) (width 0.762) (layer "F.Cu") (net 1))
 (segment (start 135.2295 80.2336) (end 135.3311 80.2336) (width 0.762) (layer "F.Cu") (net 1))
 (segment (start 137.8711 85.3136) (end 139.1411 84.0436) (width 0.762) (layer "F.Cu") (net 16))
 (segment (start 137.8711 87.8536) (end 137.8711 85.3136) (width 0.762) (layer "F.Cu") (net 16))
 (segment (start 144.2211 84.0436) (end 144.2211 81.5036) (width 0.762) (layer "F.Cu") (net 16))
 (segment (start 139.1411 84.0436) (end 144.2211 84.0436) (width 0.762) (layer "F.Cu") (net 16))
 (segment (start 155.6511 73.8836) (end 154.3811 72.6136) (width 0.762) (layer "F.Cu") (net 2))
 (segment (start 151.8411 72.6136) (end 154.3811 72.6136) (width 0.762) (layer "F.Cu") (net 2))
 (segment (start 182.3211 100.5536) (end 179.7811 100.5536) (width 0.762) (layer "F.Cu") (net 5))
 (segment (start 179.8827 96.6928) (end 182.3211 96.6928) (width 0.762) (layer "F.Cu") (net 5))
 (segment (start 183.5403 96.6928) (end 183.5911 96.7436) (width 0.762) (layer "F.Cu") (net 5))
 (segment (start 183.5403 96.6928) (end 182.3211 96.6928) (width 0.762) (layer "F.Cu") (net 5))
 (segment (start 179.7811 100.5536) (end 179.7811 105.6336) (width 0.762) (layer "F.Cu") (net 5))
 (segment (start 179.8827 96.6928) (end 179.7811 96.7436) (width 0.762) (layer "F.Cu") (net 5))
 (segment (start 182.3211 96.6928) (end 182.3211 100.5536) (width 0.762) (layer "F.Cu") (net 5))
 (segment (start 172.1103 96.6928) (end 172.1611 96.7436) (width 0.762) (layer "F.Cu") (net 6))
 (segment (start 169.6211 96.6928) (end 169.6211 105.6336) (width 0.762) (layer "F.Cu") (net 6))
 (segment (start 172.1103 96.6928) (end 169.6211 96.6928) (width 0.762) (layer "F.Cu") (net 6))
 (segment (start 168.4527 96.6928) (end 168.3511 96.7436) (width 0.762) (layer "F.Cu") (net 6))
 (segment (start 169.6211 96.6928) (end 168.4527 96.6928) (width 0.762) (layer "F.Cu") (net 6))
 (segment (start 160.6803 96.6928) (end 158.1911 96.6928) (width 0.762) (layer "F.Cu") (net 14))
 (segment (start 157.0227 96.6928) (end 156.9211 96.7436) (width 0.762) (layer "F.Cu") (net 14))
 (segment (start 160.6803 96.6928) (end 160.7311 96.7436) (width 0.762) (layer "F.Cu") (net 14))
 (segment (start 158.1911 96.6928) (end 157.0227 96.6928) (width 0.762) (layer "F.Cu") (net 14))
 (segment (start 158.1911 96.6928) (end 158.1911 105.6336) (width 0.762) (layer "F.Cu") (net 14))
 (segment (start 146.7611 96.6928) (end 146.7611 100.5536) (width 0.762) (layer "F.Cu") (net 11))
 (segment (start 146.7611 96.6928) (end 145.5927 96.6928) (width 0.762) (layer "F.Cu") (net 11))
 (segment (start 145.5927 96.6928) (end 145.4911 96.7436) (width 0.762) (layer "F.Cu") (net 11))
 (segment (start 149.2503 96.6928) (end 146.7611 96.6928) (width 0.762) (layer "F.Cu") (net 11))
 (segment (start 146.7611 100.5536) (end 149.3011 100.5536) (width 0.762) (layer "F.Cu") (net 11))
 (segment (start 149.3011 100.5536) (end 149.3011 105.6336) (width 0.762) (layer "F.Cu") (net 11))
 (segment (start 149.2503 96.6928) (end 149.3011 96.7436) (width 0.762) (layer "F.Cu") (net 11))
 (segment (start 137.8203 96.6928) (end 137.8711 96.7436) (width 0.762) (layer "F.Cu") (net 12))
 (segment (start 134.1627 96.6928) (end 134.0611 96.7436) (width 0.762) (layer "F.Cu") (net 12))
 (segment (start 136.6011 96.6928) (end 134.1627 96.6928) (width 0.762) (layer "F.Cu") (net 12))
 (segment (start 139.1411 100.5536) (end 139.1411 105.6336) (width 0.762) (layer "F.Cu") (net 12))
 (segment (start 136.6011 96.6928) (end 136.6011 100.5536) (width 0.762) (layer "F.Cu") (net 12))
 (segment (start 137.8203 96.6928) (end 136.6011 96.6928) (width 0.762) (layer "F.Cu") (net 12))
 (segment (start 136.6011 100.5536) (end 139.1411 100.5536) (width 0.762) (layer "F.Cu") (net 12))
 (segment (start 126.3903 96.6928) (end 123.9011 96.6928) (width 0.762) (layer "F.Cu") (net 17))
 (segment (start 128.9811 101.8236) (end 128.9811 105.6336) (width 0.762) (layer "F.Cu") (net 17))
 (segment (start 123.9011 96.6928) (end 122.7327 96.6928) (width 0.762) (layer "F.Cu") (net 17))
 (segment (start 123.9011 101.8236) (end 128.9811 101.8236) (width 0.762) (layer "F.Cu") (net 17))
 (segment (start 122.7327 96.6928) (end 122.6311 96.7436) (width 0.762) (layer "F.Cu") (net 17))
 (segment (start 126.3903 96.6928) (end 126.4411 96.7436) (width 0.762) (layer "F.Cu") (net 17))
 (segment (start 123.9011 96.6928) (end 123.9011 101.8236) (width 0.762) (layer "F.Cu") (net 17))
 (segment (start 114.9603 96.6928) (end 112.4711 96.6928) (width 0.762) (layer "F.Cu") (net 3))
 (segment (start 114.9603 96.6928) (end 115.0111 96.7436) (width 0.762) (layer "F.Cu") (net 3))
 (segment (start 112.4711 96.6928) (end 111.3027 96.6928) (width 0.762) (layer "F.Cu") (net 3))
 (segment (start 112.4711 96.6928) (end 112.4711 101.8236) (width 0.762) (layer "F.Cu") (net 3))
 (segment (start 111.3027 96.6928) (end 111.2011 96.7436) (width 0.762) (layer "F.Cu") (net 3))
 (segment (start 112.4711 101.8236) (end 117.5511 101.8236) (width 0.762) (layer "F.Cu") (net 3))
 (segment (start 117.5511 101.8236) (end 117.5511 105.6336) (width 0.762) (layer "F.Cu") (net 3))
 (segment (start 103.5811 96.7436) (end 103.5811 101.8236) (width 0.762) (layer "F.Cu") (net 4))
 (segment (start 107.3911 101.8236) (end 107.3911 106.9036) (width 0.762) (layer "F.Cu") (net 4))
 (segment (start 103.5811 101.8236) (end 107.3911 101.8236) (width 0.762) (layer "F.Cu") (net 4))
 (segment (start 191.2111 96.7436) (end 191.2111 105.6336) (width 0.762) (layer "F.Cu") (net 13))
 (segment (start 191.2111 81.5036) (end 191.2111 96.7436) (width 0.762) (layer "F.Cu") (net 13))
 (segment (start 155.6511 81.5036) (end 191.2111 81.5036) (width 0.762) (layer "F.Cu") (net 13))
 (segment (start 151.8411 81.5036) (end 151.8411 77.6936) (width 0.762) (layer "F.Cu") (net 7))
 (segment (start 151.8411 77.6936) (end 159.4611 77.6936) (width 0.762) (layer "F.Cu") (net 7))
 (segment (start 159.4611 77.6936) (end 181.0511 77.6936) (width 0.762) (layer "F.Cu") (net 7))
 (segment (start 159.4611 75.1536) (end 167.6399 75.1536) (width 0.762) (layer "F.Cu") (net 8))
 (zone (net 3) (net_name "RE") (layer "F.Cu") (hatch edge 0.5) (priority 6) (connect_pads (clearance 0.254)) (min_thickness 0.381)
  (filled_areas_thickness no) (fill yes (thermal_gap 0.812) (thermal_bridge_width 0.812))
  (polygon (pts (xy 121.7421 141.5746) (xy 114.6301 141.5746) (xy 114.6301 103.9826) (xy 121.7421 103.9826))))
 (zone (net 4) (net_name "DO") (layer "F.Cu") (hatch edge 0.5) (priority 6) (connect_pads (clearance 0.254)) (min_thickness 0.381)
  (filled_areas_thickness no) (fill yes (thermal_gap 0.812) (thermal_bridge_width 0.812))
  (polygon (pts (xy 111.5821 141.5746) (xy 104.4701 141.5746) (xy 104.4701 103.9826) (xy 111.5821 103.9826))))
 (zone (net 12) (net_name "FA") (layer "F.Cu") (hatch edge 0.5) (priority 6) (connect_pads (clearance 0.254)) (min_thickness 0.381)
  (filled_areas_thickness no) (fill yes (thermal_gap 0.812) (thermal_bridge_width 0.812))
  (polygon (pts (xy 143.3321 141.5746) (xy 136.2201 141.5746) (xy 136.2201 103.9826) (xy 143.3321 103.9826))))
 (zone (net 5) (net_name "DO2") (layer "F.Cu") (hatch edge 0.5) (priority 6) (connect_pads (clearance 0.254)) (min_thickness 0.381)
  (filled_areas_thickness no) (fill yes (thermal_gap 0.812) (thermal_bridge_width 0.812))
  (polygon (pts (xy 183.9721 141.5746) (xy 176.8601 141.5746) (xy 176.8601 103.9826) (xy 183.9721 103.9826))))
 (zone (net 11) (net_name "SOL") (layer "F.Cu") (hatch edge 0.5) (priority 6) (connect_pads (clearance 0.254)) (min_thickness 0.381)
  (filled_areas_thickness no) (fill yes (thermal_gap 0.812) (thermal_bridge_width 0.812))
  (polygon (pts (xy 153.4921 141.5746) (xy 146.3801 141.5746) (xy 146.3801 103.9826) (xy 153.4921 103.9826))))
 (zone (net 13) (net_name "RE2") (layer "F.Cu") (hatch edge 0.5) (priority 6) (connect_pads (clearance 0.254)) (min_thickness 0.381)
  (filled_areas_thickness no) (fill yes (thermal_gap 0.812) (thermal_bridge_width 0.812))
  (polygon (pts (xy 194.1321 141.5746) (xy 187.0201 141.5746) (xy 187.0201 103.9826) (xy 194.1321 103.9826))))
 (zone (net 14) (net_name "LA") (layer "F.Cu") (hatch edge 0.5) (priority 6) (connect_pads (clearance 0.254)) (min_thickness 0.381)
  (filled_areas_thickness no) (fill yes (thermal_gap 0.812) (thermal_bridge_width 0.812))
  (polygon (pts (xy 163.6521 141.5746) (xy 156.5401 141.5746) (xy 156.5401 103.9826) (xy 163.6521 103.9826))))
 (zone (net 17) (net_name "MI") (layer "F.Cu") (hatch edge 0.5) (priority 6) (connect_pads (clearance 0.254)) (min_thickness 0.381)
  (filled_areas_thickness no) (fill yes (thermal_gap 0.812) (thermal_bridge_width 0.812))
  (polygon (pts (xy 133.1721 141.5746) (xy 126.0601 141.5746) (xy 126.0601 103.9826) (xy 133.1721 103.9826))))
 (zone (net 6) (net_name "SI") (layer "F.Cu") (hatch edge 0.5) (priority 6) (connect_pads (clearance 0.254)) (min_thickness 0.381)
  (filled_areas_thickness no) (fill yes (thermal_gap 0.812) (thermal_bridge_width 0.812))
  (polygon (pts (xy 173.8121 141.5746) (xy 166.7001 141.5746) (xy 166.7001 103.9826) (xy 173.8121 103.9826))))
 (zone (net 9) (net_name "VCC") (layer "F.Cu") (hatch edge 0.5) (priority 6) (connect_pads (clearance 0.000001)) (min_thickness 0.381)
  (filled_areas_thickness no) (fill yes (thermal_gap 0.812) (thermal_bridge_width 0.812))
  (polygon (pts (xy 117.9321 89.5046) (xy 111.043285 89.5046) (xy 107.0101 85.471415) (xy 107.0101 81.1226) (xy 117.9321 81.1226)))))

